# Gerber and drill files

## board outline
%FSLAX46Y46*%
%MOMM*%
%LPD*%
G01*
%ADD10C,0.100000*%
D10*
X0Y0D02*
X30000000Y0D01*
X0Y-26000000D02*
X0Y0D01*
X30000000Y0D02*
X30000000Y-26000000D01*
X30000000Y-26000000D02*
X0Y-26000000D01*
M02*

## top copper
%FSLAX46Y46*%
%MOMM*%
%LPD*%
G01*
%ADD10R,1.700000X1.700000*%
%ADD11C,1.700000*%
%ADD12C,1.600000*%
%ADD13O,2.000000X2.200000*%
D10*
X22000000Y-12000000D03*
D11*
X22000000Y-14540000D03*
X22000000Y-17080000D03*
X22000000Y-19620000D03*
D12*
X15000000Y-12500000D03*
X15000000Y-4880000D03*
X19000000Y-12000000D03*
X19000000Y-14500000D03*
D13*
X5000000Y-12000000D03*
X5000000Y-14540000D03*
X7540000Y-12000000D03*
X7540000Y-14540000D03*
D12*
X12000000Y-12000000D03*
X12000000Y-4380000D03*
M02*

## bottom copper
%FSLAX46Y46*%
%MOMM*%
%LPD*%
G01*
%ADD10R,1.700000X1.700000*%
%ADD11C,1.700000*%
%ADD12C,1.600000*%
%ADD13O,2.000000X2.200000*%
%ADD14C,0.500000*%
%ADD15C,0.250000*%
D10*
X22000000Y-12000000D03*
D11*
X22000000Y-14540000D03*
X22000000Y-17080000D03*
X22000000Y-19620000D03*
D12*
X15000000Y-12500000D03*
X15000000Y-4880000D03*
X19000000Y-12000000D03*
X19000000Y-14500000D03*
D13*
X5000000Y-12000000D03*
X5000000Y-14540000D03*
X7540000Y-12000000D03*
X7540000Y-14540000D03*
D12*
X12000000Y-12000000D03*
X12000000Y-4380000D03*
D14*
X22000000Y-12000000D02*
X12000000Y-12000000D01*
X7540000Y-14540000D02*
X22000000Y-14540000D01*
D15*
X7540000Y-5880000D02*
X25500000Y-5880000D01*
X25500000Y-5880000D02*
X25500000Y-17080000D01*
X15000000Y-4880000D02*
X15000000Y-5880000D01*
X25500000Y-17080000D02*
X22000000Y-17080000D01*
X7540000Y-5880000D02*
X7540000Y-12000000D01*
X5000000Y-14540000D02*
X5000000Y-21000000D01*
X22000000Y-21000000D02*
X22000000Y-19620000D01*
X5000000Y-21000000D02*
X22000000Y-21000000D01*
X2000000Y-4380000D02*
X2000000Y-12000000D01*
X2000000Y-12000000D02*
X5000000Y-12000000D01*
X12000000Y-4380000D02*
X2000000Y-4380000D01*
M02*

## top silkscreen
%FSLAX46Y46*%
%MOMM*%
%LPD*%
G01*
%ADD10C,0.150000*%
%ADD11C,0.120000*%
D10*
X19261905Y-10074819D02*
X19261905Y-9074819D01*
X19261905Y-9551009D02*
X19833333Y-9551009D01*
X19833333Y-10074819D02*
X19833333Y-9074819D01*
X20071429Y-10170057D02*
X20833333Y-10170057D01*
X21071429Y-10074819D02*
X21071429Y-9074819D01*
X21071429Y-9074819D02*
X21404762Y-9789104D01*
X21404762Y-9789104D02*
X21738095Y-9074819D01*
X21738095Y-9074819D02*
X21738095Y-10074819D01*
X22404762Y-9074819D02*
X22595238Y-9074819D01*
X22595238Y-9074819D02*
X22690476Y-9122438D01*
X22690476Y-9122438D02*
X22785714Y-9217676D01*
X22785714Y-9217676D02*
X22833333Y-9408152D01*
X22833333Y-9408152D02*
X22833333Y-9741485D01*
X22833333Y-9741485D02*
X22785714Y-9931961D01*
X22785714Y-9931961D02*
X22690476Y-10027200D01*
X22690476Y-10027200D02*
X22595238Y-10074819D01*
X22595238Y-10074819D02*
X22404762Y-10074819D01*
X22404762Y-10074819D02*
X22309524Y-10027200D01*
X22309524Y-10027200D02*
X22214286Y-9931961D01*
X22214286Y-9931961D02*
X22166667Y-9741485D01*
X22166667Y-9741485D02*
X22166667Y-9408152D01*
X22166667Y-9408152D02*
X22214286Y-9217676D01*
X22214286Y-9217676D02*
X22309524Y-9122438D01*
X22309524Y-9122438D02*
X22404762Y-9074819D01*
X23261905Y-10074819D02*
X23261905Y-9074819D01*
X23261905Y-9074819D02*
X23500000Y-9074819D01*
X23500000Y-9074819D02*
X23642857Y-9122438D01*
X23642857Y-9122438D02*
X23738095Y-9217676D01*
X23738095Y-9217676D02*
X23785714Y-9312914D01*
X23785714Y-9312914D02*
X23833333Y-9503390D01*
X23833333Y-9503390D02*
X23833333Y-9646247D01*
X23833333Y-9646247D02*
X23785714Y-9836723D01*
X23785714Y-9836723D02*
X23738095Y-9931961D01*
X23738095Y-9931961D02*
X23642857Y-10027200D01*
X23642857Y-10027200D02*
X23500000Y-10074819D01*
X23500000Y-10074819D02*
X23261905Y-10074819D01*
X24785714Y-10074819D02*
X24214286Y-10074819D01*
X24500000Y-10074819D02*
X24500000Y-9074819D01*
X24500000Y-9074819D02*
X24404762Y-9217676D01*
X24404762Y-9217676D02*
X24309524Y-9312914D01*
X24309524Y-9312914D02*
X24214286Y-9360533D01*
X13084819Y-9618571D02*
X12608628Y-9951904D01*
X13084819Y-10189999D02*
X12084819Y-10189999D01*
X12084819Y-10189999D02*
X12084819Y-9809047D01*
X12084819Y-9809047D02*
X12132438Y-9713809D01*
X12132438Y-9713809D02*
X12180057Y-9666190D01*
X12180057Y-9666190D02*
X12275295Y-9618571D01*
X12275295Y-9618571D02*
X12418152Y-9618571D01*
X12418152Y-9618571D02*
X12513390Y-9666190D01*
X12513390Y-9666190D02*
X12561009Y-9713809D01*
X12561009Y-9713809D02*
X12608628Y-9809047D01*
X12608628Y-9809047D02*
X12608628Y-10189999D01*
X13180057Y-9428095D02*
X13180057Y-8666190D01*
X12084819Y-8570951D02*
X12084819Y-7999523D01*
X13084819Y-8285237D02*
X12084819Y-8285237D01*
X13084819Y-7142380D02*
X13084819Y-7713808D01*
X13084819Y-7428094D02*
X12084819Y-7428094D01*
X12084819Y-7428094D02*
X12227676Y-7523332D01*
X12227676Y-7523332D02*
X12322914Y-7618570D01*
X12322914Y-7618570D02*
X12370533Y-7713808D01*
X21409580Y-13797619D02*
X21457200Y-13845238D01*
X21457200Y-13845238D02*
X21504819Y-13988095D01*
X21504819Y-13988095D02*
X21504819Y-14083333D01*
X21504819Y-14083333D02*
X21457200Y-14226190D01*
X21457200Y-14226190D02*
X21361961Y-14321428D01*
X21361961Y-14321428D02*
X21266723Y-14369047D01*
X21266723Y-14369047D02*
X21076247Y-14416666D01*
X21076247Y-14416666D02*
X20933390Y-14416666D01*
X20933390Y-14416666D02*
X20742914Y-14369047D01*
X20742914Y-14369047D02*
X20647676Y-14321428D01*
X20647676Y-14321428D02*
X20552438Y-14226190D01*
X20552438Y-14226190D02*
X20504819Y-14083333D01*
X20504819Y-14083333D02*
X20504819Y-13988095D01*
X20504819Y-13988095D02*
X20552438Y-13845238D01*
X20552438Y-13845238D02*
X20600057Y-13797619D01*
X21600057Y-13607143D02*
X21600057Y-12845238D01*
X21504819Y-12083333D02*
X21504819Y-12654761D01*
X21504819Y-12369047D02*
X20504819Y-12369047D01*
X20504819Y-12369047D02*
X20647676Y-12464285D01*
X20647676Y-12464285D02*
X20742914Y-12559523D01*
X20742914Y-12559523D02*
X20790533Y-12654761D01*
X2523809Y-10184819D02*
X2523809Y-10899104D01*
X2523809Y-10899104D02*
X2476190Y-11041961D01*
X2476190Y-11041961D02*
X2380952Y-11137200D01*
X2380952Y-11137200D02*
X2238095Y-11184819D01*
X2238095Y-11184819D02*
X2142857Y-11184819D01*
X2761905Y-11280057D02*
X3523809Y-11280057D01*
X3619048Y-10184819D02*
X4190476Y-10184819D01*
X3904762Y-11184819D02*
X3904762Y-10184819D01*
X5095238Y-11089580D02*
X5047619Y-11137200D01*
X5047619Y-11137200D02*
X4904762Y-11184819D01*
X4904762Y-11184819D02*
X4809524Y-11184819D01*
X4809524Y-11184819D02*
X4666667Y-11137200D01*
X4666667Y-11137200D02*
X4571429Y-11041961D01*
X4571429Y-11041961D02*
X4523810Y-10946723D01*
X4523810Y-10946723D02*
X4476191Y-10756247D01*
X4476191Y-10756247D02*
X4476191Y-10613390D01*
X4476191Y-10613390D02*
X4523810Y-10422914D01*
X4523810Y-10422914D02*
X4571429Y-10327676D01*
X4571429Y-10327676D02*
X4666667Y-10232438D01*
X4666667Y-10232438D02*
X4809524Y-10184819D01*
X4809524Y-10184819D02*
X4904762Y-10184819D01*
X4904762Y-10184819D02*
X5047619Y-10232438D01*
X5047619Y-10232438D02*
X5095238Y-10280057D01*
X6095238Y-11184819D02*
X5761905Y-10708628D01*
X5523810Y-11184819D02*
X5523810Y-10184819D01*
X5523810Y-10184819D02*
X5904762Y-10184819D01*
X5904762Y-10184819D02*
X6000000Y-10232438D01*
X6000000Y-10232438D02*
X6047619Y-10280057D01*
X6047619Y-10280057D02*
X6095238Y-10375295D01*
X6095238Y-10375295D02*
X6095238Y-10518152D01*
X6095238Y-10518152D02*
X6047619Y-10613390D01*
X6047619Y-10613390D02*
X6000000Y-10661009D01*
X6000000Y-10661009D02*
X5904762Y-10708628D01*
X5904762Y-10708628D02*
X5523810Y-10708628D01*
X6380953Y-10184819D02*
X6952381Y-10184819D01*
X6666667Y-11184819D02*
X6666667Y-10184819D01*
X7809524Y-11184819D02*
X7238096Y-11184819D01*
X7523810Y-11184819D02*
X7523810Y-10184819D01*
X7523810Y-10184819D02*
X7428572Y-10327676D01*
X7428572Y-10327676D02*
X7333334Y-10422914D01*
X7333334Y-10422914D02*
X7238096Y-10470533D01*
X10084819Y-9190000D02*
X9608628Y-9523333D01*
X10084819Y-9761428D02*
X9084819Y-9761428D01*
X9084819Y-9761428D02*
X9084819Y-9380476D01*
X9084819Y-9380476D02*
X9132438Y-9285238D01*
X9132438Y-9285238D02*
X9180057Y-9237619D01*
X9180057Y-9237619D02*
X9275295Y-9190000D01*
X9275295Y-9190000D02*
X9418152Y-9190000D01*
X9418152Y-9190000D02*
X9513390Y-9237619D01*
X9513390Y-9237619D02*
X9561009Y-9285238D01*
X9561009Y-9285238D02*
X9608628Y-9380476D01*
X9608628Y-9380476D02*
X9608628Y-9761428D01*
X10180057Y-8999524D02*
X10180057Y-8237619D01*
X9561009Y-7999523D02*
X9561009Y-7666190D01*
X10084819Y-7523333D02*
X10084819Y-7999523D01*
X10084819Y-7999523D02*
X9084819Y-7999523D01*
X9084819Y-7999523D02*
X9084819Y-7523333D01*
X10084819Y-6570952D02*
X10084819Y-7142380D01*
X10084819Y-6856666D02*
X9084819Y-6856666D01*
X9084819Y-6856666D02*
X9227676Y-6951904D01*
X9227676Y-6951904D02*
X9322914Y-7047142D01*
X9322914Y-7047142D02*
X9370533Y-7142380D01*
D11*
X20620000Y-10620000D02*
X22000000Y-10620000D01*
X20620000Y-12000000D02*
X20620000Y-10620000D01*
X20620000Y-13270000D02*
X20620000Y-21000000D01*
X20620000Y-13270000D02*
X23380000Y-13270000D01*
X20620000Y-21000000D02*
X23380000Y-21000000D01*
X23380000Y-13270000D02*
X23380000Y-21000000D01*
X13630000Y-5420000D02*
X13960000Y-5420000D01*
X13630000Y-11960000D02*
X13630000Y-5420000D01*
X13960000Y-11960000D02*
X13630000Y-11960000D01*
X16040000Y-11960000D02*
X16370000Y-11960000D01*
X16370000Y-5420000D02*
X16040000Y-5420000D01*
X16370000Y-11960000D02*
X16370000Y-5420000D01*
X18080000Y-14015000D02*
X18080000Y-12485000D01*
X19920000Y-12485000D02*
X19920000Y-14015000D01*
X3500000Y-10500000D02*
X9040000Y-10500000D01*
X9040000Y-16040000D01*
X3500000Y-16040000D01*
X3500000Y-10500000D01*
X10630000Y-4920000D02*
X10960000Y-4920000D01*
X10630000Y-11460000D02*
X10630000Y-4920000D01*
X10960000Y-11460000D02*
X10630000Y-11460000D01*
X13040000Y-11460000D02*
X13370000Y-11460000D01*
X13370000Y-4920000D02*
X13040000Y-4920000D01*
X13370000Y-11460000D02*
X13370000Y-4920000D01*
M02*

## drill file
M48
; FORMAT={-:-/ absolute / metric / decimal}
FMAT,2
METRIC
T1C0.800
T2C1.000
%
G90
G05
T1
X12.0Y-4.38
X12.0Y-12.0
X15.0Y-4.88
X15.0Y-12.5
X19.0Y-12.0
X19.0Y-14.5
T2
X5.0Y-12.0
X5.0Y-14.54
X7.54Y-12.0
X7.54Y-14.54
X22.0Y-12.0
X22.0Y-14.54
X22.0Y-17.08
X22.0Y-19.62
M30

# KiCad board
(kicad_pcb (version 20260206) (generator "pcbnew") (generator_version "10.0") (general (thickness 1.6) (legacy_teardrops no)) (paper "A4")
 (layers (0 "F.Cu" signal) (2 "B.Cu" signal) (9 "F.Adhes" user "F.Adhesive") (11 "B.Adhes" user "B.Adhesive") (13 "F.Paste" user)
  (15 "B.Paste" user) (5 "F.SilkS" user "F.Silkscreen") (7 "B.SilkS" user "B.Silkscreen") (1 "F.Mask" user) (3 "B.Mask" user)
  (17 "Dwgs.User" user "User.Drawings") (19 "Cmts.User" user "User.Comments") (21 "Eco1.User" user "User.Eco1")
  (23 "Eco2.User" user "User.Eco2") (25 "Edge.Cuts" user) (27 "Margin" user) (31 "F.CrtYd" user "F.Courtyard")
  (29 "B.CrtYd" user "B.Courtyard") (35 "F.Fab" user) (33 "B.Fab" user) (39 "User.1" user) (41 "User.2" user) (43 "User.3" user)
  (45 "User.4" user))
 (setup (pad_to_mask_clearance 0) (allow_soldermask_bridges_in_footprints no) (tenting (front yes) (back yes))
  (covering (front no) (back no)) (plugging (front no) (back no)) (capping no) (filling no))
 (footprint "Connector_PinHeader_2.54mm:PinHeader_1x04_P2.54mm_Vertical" (layer "F.Cu") (at 22 12)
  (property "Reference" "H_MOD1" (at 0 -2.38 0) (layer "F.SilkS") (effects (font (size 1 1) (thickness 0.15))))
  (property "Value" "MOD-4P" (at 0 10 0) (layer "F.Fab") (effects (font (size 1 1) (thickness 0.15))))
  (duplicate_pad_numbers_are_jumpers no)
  (fp_line (start -1.38 -1.38) (end 0 -1.38) (stroke (width 0.12) (type solid)) (layer "F.SilkS"))
  (fp_line (start -1.38 0) (end -1.38 -1.38) (stroke (width 0.12) (type solid)) (layer "F.SilkS"))
  (fp_line (start -1.38 1.27) (end -1.38 9) (stroke (width 0.12) (type solid)) (layer "F.SilkS"))
  (fp_line (start -1.38 1.27) (end 1.38 1.27) (stroke (width 0.12) (type solid)) (layer "F.SilkS"))
  (fp_line (start -1.38 9) (end 1.38 9) (stroke (width 0.12) (type solid)) (layer "F.SilkS"))
  (fp_line (start 1.38 1.27) (end 1.38 9) (stroke (width 0.12) (type solid)) (layer "F.SilkS"))
  (pad "1" thru_hole rect (at 0 0) (size 1.7 1.7) (drill 1) (layers "*.Cu" "*.Mask") (remove_unused_layers no) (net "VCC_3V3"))
  (pad "2" thru_hole circle (at 0 2.54) (size 1.7 1.7) (drill 1) (layers "*.Cu" "*.Mask") (remove_unused_layers no) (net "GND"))
  (pad "3" thru_hole circle (at 0 5.08) (size 1.7 1.7) (drill 1) (layers "*.Cu" "*.Mask") (remove_unused_layers no) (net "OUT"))
  (pad "4" thru_hole circle (at 0 7.62) (size 1.7 1.7) (drill 1) (layers "*.Cu" "*.Mask") (remove_unused_layers no) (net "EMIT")))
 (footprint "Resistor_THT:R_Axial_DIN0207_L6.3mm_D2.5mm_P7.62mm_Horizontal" (layer "F.Cu") (at 15 12.5 90)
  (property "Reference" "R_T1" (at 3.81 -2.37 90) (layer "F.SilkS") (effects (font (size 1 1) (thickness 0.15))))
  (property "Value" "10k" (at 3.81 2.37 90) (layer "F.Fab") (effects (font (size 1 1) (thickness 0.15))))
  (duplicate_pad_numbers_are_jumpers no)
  (fp_line (start 7.08 -1.37) (end 7.08 -1.04) (stroke (width 0.12) (type solid)) (layer "F.SilkS"))
  (fp_line (start 0.54 -1.37) (end 7.08 -1.37) (stroke (width 0.12) (type solid)) (layer "F.SilkS"))
  (fp_line (start 0.54 -1.04) (end 0.54 -1.37) (stroke (width 0.12) (type solid)) (layer "F.SilkS"))
  (fp_line (start 0.54 1.04) (end 0.54 1.37) (stroke (width 0.12) (type solid)) (layer "F.SilkS"))
  (fp_line (start 7.08 1.37) (end 7.08 1.04) (stroke (width 0.12) (type solid)) (layer "F.SilkS"))
  (fp_line (start 0.54 1.37) (end 7.08 1.37) (stroke (width 0.12) (type solid)) (layer "F.SilkS"))
  (pad "1" thru_hole circle (at 0 0 90) (size 1.6 1.6) (drill 0.8) (layers "*.Cu" "*.Mask") (remove_unused_layers no) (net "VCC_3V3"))
  (pad "2" thru_hole circle (at 7.62 0 90) (size 1.6 1.6) (drill 0.8) (layers "*.Cu" "*.Mask") (remove_unused_layers no) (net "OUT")))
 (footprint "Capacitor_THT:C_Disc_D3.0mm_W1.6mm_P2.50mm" (layer "F.Cu") (at 19 12 -90)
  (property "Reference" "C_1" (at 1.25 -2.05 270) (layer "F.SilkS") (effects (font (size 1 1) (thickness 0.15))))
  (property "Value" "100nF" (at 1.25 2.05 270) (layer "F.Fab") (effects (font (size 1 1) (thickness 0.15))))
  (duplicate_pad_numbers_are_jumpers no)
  (fp_line (start 2.015 0.92) (end 0.485 0.92) (stroke (width 0.12) (type solid)) (layer "F.SilkS"))
  (fp_line (start 0.485 -0.92) (end 2.015 -0.92) (stroke (width 0.12) (type solid)) (layer "F.SilkS"))
  (pad "1" thru_hole circle (at 0 0 270) (size 1.6 1.6) (drill 0.8) (layers "*.Cu" "*.Mask") (remove_unused_layers no) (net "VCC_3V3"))
  (pad "2" thru_hole circle (at 2.5 0 270) (size 1.6 1.6) (drill 0.8) (layers "*.Cu" "*.Mask") (remove_unused_layers no) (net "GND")))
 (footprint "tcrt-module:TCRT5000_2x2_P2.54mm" (layer "F.Cu") (at 5 12)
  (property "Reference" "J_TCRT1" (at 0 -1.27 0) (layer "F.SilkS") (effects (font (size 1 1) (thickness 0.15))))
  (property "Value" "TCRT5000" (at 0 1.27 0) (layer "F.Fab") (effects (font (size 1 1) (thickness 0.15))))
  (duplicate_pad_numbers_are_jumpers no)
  (fp_rect (start -1.5 -1.5) (end 4.04 4.04) (stroke (width 0.12) (type default)) (fill no) (layer "F.SilkS"))
  (pad "1" thru_hole oval (at 0 0) (size 2 2.2) (drill 1) (layers "*.Cu" "*.Mask") (remove_unused_layers no) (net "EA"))
  (pad "2" thru_hole oval (at 0 2.54) (size 2 2.2) (drill 1) (layers "*.Cu" "*.Mask") (remove_unused_layers no) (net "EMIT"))
  (pad "3" thru_hole oval (at 2.54 0) (size 2 2.2) (drill 1) (layers "*.Cu" "*.Mask") (remove_unused_layers no) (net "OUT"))
  (pad "4" thru_hole oval (at 2.54 2.54) (size 2 2.2) (drill 1) (layers "*.Cu" "*.Mask") (remove_unused_layers no) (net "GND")))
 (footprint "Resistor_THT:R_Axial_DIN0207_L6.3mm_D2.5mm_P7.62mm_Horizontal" (layer "F.Cu") (at 12 12 90)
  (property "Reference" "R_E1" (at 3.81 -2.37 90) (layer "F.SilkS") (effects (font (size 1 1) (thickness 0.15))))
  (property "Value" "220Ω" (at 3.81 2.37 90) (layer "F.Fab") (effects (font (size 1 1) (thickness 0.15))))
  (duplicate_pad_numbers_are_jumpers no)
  (fp_line (start 7.08 -1.37) (end 7.08 -1.04) (stroke (width 0.12) (type solid)) (layer "F.SilkS"))
  (fp_line (start 0.54 -1.37) (end 7.08 -1.37) (stroke (width 0.12) (type solid)) (layer "F.SilkS"))
  (fp_line (start 0.54 -1.04) (end 0.54 -1.37) (stroke (width 0.12) (type solid)) (layer "F.SilkS"))
  (fp_line (start 0.54 1.04) (end 0.54 1.37) (stroke (width 0.12) (type solid)) (layer "F.SilkS"))
  (fp_line (start 7.08 1.37) (end 7.08 1.04) (stroke (width 0.12) (type solid)) (layer "F.SilkS"))
  (fp_line (start 0.54 1.37) (end 7.08 1.37) (stroke (width 0.12) (type solid)) (layer "F.SilkS"))
  (pad "1" thru_hole circle (at 0 0 90) (size 1.6 1.6) (drill 0.8) (layers "*.Cu" "*.Mask") (remove_unused_layers no) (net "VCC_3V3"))
  (pad "2" thru_hole circle (at 7.62 0 90) (size 1.6 1.6) (drill 0.8) (layers "*.Cu" "*.Mask") (remove_unused_layers no) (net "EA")))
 (gr_line (start 0 0) (end 30 0) (stroke (width 0) (type default)) (layer "Edge.Cuts"))
 (gr_line (start 0 26) (end 0 0) (stroke (width 0) (type default)) (layer "Edge.Cuts"))
 (gr_line (start 30 0) (end 30 26) (stroke (width 0) (type default)) (layer "Edge.Cuts"))
 (gr_line (start 30 26) (end 0 26) (stroke (width 0) (type default)) (layer "Edge.Cuts"))
 (segment (start 22 12) (end 12 12) (width 0.5) (layer "B.Cu") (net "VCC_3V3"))
 (segment (start 7.54 14.54) (end 22 14.54) (width 0.5) (layer "B.Cu") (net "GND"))
 (segment (start 7.54 5.88) (end 25.5 5.88) (width 0.25) (layer "B.Cu") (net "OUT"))
 (segment (start 25.5 5.88) (end 25.5 17.08) (width 0.25) (layer "B.Cu") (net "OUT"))
 (segment (start 15 4.88) (end 15 5.88) (width 0.25) (layer "B.Cu") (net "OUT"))
 (segment (start 25.5 17.08) (end 22 17.08) (width 0.25) (layer "B.Cu") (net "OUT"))
 (segment (start 7.54 5.88) (end 7.54 12) (width 0.25) (layer "B.Cu") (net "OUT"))
 (segment (start 5 14.54) (end 5 21) (width 0.25) (layer "B.Cu") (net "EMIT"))
 (segment (start 22 21) (end 22 19.62) (width 0.25) (layer "B.Cu") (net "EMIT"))
 (segment (start 5 21) (end 22 21) (width 0.25) (layer "B.Cu") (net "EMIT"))
 (segment (start 2 4.38) (end 2 12) (width 0.25) (layer "B.Cu") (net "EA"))
 (segment (start 2 12) (end 5 12) (width 0.25) (layer "B.Cu") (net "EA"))
 (segment (start 12 4.38) (end 2 4.38) (width 0.25) (layer "B.Cu") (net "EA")))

